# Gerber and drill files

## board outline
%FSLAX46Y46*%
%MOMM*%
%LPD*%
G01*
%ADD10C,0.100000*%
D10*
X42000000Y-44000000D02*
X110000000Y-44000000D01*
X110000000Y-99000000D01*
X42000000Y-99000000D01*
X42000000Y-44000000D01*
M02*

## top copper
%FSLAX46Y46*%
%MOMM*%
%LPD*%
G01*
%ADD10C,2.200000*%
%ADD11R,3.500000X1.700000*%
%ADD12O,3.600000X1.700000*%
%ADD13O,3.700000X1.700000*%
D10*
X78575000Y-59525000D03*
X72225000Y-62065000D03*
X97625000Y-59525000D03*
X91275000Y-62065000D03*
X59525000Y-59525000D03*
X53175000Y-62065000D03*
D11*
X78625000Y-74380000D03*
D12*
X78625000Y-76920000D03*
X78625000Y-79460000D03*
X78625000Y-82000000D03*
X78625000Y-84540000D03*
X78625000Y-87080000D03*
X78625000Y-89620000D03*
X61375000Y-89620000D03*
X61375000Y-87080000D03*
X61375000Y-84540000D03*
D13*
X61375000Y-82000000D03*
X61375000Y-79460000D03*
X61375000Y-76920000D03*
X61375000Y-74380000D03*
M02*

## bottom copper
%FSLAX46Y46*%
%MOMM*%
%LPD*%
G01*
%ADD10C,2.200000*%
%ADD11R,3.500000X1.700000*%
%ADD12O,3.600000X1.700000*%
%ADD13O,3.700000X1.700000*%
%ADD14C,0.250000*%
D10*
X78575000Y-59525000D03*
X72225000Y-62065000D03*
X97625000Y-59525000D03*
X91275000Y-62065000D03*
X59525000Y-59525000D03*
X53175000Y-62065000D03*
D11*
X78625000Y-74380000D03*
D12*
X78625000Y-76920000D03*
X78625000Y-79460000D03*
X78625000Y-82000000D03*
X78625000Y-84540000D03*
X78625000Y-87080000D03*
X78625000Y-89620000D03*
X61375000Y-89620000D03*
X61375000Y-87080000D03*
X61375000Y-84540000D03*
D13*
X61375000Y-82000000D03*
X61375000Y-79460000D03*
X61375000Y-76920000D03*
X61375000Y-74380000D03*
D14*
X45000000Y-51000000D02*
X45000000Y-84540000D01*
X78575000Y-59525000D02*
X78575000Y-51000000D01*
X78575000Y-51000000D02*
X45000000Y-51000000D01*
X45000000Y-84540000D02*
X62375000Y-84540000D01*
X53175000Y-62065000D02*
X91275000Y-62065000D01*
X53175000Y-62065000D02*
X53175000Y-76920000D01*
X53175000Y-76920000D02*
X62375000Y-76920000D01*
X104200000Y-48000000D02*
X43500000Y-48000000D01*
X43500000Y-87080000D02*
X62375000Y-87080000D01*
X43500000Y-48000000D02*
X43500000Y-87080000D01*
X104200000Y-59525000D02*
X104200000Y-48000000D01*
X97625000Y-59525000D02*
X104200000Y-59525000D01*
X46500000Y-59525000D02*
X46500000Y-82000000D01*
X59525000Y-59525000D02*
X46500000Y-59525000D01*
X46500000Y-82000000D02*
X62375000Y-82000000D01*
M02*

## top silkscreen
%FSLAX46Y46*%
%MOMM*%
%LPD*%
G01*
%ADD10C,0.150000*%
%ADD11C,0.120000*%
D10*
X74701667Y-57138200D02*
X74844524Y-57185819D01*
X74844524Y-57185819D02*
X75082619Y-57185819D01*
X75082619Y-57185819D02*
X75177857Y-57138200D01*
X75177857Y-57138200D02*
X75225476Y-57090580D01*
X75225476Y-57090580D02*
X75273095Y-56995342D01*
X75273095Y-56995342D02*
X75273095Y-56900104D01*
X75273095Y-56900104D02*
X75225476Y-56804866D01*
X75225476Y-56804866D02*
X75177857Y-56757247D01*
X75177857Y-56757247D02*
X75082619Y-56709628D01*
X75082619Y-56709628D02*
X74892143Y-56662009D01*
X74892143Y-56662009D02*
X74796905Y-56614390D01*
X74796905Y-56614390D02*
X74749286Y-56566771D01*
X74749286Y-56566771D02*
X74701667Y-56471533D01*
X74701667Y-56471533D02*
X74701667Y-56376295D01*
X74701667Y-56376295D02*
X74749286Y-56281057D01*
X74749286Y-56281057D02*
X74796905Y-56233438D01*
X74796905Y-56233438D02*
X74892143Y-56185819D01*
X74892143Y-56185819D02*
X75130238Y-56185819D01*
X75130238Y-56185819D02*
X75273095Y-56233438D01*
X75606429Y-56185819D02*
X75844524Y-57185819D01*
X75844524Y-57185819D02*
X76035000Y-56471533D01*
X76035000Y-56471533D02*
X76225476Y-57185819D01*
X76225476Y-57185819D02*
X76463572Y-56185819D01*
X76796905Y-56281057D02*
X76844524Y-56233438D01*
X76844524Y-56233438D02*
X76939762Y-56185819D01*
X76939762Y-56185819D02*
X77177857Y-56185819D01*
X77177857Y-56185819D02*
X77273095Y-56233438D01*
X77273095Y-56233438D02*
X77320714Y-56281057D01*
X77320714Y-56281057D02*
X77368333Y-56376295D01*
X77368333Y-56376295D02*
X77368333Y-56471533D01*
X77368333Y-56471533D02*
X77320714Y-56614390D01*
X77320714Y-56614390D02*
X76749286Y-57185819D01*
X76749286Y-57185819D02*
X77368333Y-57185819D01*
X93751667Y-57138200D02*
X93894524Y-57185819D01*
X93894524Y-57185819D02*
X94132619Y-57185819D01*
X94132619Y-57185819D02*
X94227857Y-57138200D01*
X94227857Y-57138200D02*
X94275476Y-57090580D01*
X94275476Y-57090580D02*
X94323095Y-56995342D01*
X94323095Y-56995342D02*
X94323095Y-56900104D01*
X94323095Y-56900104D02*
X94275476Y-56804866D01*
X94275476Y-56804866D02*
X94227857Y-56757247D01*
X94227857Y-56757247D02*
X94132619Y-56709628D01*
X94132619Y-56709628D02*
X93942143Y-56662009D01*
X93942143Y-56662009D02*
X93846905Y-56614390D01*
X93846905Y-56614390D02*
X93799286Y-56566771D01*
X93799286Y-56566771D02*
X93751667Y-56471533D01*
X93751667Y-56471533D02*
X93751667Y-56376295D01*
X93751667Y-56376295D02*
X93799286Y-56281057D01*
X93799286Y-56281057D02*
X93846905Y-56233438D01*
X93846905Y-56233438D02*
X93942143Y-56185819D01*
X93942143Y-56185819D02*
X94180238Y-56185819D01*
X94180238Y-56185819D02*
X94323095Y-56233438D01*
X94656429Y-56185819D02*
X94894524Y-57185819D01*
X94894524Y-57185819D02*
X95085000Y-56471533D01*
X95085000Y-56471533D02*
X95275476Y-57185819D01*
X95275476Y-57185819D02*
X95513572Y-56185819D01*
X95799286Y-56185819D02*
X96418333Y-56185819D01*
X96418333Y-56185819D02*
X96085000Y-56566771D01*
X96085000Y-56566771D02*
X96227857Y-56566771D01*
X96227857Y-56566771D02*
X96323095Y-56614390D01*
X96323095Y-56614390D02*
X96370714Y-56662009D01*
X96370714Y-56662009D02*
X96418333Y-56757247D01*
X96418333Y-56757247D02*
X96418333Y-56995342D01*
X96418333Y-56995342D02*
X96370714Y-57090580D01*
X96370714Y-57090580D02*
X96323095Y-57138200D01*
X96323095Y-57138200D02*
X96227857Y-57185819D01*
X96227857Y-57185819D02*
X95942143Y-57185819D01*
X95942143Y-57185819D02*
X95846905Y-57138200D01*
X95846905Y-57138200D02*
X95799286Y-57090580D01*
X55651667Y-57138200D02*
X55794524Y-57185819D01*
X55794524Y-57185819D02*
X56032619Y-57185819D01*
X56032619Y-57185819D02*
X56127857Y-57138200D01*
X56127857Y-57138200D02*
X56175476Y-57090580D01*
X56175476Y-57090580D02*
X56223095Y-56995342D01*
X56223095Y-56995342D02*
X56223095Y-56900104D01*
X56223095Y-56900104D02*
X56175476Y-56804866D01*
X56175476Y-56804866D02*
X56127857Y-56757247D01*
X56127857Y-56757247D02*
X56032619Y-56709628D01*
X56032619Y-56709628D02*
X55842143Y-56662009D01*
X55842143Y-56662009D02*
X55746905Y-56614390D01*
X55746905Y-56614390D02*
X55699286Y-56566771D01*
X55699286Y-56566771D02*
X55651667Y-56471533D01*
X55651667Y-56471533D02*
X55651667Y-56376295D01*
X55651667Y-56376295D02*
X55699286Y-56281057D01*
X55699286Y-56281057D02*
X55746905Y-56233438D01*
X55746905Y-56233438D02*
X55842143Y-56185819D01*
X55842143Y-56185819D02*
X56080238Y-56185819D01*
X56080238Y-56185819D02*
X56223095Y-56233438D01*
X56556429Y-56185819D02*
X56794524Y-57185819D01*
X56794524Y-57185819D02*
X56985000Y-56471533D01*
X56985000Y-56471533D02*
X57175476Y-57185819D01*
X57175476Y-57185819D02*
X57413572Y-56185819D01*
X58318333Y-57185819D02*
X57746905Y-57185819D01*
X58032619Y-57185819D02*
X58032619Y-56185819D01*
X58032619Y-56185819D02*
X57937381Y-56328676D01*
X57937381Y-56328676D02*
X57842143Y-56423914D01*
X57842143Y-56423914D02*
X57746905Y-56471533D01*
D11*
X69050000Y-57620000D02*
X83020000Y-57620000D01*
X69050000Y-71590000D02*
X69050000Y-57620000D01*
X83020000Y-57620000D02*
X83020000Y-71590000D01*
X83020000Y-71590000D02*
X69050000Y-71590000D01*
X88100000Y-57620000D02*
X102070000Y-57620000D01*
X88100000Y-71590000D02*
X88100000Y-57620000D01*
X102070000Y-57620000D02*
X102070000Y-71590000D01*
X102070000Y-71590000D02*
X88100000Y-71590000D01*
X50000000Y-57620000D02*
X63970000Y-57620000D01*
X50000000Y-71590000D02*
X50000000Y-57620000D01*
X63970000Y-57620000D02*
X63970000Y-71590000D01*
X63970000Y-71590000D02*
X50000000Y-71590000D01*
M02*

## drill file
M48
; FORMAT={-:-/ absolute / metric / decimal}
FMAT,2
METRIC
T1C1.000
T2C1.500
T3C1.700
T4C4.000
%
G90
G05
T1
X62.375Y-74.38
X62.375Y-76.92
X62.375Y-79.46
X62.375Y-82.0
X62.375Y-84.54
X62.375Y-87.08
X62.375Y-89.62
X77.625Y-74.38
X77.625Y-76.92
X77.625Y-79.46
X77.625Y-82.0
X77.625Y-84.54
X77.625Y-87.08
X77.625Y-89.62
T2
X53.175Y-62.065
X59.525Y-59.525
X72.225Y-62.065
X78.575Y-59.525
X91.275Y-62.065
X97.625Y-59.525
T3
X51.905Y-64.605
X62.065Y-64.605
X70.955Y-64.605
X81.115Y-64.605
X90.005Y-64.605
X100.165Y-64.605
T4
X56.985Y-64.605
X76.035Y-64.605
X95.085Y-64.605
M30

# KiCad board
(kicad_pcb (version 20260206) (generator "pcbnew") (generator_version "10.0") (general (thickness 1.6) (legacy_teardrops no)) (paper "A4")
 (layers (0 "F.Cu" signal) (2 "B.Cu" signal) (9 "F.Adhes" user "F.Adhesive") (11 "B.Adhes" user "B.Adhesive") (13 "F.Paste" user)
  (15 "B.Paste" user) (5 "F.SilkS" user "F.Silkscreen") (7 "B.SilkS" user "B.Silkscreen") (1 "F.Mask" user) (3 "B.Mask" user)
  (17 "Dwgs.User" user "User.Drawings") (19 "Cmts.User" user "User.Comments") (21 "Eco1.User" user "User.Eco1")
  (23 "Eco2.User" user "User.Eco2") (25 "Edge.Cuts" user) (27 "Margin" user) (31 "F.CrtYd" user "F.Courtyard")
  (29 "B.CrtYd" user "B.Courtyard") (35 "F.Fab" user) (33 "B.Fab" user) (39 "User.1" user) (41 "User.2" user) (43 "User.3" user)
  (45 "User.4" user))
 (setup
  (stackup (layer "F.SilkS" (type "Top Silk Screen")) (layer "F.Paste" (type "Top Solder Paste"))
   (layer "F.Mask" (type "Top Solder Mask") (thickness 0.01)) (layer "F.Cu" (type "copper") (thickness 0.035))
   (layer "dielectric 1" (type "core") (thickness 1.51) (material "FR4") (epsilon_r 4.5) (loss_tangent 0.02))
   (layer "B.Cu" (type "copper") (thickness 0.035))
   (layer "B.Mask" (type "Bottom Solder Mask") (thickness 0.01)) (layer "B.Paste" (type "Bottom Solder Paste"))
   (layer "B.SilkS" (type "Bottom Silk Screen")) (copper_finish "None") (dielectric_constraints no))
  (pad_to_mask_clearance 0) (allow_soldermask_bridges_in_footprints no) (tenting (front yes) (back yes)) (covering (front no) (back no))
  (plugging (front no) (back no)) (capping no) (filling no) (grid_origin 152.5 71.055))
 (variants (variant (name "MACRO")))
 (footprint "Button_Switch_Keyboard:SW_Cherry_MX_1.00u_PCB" (layer "F.Cu") (at 78.575 59.525)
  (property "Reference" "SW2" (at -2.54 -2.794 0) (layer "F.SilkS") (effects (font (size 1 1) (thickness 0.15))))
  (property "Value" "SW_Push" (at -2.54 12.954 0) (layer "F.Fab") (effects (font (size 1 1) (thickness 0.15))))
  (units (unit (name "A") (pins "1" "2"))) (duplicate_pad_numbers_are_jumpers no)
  (fp_line (start -9.525 -1.905) (end 4.445 -1.905) (stroke (width 0.12) (type solid)) (layer "F.SilkS"))
  (fp_line (start -9.525 12.065) (end -9.525 -1.905) (stroke (width 0.12) (type solid)) (layer "F.SilkS"))
  (fp_line (start 4.445 -1.905) (end 4.445 12.065) (stroke (width 0.12) (type solid)) (layer "F.SilkS"))
  (fp_line (start 4.445 12.065) (end -9.525 12.065) (stroke (width 0.12) (type solid)) (layer "F.SilkS"))
  (pad "" np_thru_hole circle (at -7.62 5.08) (size 1.7 1.7) (drill 1.7) (layers "*.Cu" "*.Mask"))
  (pad "" np_thru_hole circle (at -2.54 5.08) (size 4 4) (drill 4) (layers "*.Cu" "*.Mask"))
  (pad "" np_thru_hole circle (at 2.54 5.08) (size 1.7 1.7) (drill 1.7) (layers "*.Cu" "*.Mask"))
  (pad "1" thru_hole circle (at 0 0) (size 2.2 2.2) (drill 1.5) (layers "*.Cu" "*.Mask") (remove_unused_layers no)
   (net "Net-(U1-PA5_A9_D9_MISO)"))
  (pad "2" thru_hole circle (at -6.35 2.54) (size 2.2 2.2) (drill 1.5) (layers "*.Cu" "*.Mask") (remove_unused_layers no) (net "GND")))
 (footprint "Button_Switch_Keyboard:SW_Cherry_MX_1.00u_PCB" (layer "F.Cu") (at 97.625 59.525)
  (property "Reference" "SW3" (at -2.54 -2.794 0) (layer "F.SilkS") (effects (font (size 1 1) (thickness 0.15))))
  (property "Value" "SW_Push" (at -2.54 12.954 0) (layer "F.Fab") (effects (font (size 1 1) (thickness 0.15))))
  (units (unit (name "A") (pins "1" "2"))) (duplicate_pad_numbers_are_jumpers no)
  (fp_line (start -9.525 -1.905) (end 4.445 -1.905) (stroke (width 0.12) (type solid)) (layer "F.SilkS"))
  (fp_line (start -9.525 12.065) (end -9.525 -1.905) (stroke (width 0.12) (type solid)) (layer "F.SilkS"))
  (fp_line (start 4.445 -1.905) (end 4.445 12.065) (stroke (width 0.12) (type solid)) (layer "F.SilkS"))
  (fp_line (start 4.445 12.065) (end -9.525 12.065) (stroke (width 0.12) (type solid)) (layer "F.SilkS"))
  (pad "" np_thru_hole circle (at -7.62 5.08) (size 1.7 1.7) (drill 1.7) (layers "*.Cu" "*.Mask"))
  (pad "" np_thru_hole circle (at -2.54 5.08) (size 4 4) (drill 4) (layers "*.Cu" "*.Mask"))
  (pad "" np_thru_hole circle (at 2.54 5.08) (size 1.7 1.7) (drill 1.7) (layers "*.Cu" "*.Mask"))
  (pad "1" thru_hole circle (at 0 0) (size 2.2 2.2) (drill 1.5) (layers "*.Cu" "*.Mask") (remove_unused_layers no)
   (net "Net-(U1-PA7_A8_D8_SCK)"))
  (pad "2" thru_hole circle (at -6.35 2.54) (size 2.2 2.2) (drill 1.5) (layers "*.Cu" "*.Mask") (remove_unused_layers no) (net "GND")))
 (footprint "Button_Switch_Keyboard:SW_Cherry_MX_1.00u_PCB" (layer "F.Cu") (at 59.525 59.525)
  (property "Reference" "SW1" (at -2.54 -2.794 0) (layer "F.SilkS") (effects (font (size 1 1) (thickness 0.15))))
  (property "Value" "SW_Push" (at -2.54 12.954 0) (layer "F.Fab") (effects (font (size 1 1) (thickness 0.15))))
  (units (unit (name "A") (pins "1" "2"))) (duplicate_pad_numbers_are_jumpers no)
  (fp_line (start -9.525 -1.905) (end 4.445 -1.905) (stroke (width 0.12) (type solid)) (layer "F.SilkS"))
  (fp_line (start -9.525 12.065) (end -9.525 -1.905) (stroke (width 0.12) (type solid)) (layer "F.SilkS"))
  (fp_line (start 4.445 -1.905) (end 4.445 12.065) (stroke (width 0.12) (type solid)) (layer "F.SilkS"))
  (fp_line (start 4.445 12.065) (end -9.525 12.065) (stroke (width 0.12) (type solid)) (layer "F.SilkS"))
  (pad "" np_thru_hole circle (at -7.62 5.08) (size 1.7 1.7) (drill 1.7) (layers "*.Cu" "*.Mask"))
  (pad "" np_thru_hole circle (at -2.54 5.08) (size 4 4) (drill 4) (layers "*.Cu" "*.Mask"))
  (pad "" np_thru_hole circle (at 2.54 5.08) (size 1.7 1.7) (drill 1.7) (layers "*.Cu" "*.Mask"))
  (pad "1" thru_hole circle (at 0 0) (size 2.2 2.2) (drill 1.5) (layers "*.Cu" "*.Mask") (remove_unused_layers no)
   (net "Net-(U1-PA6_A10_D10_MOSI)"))
  (pad "2" thru_hole circle (at -6.35 2.54) (size 2.2 2.2) (drill 1.5) (layers "*.Cu" "*.Mask") (remove_unused_layers no) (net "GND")))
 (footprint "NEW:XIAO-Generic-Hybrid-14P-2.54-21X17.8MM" (layer "B.Cu") (at 70 82 180)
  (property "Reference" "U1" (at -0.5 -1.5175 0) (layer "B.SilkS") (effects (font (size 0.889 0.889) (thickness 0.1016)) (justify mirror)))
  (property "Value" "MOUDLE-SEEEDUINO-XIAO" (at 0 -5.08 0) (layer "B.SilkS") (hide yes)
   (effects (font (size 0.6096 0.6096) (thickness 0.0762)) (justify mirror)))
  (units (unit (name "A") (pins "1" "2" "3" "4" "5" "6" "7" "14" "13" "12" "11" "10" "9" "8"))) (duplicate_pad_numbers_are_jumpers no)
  (pad "1" thru_hole rect (at -7.625 7.62 180) (size 3.5 1.7) (drill 1 (offset -1 0)) (layers "*.Cu" "*.Mask") (remove_unused_layers no)
   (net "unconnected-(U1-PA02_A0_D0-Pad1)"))
  (pad "2" thru_hole oval (at -7.625 5.08 180) (size 3.6 1.7) (drill 1 (offset -1 0)) (layers "*.Cu" "*.Mask") (remove_unused_layers no)
   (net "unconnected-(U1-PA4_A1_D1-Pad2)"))
  (pad "3" thru_hole oval (at -7.625 2.54 180) (size 3.6 1.7) (drill 1 (offset -1 0)) (layers "*.Cu" "*.Mask") (remove_unused_layers no)
   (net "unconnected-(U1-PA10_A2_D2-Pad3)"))
  (pad "4" thru_hole oval (at -7.625 0 180) (size 3.6 1.7) (drill 1 (offset -1 0)) (layers "*.Cu" "*.Mask") (remove_unused_layers no)
   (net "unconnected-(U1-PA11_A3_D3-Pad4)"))
  (pad "5" thru_hole oval (at -7.625 -2.54 180) (size 3.6 1.7) (drill 1 (offset -1 0)) (layers "*.Cu" "*.Mask") (remove_unused_layers no)
   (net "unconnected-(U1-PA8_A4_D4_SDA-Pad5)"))
  (pad "6" thru_hole oval (at -7.625 -5.08) (size 3.6 1.7) (drill 1 (offset 1 0)) (layers "*.Cu" "*.Mask") (remove_unused_layers no)
   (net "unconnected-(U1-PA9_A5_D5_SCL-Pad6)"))
  (pad "7" thru_hole oval (at -7.625 -7.62 180) (size 3.6 1.7) (drill 1 (offset -1 0)) (layers "*.Cu" "*.Mask") (remove_unused_layers no)
   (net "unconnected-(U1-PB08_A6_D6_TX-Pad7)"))
  (pad "8" thru_hole oval (at 7.625 -7.62 180) (size 3.6 1.7) (drill 1 (offset 1 0)) (layers "*.Cu" "*.Mask") (remove_unused_layers no)
   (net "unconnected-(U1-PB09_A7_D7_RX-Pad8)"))
  (pad "9" thru_hole oval (at 7.625 -5.08 180) (size 3.6 1.7) (drill 1 (offset 1 0)) (layers "*.Cu" "*.Mask") (remove_unused_layers no)
   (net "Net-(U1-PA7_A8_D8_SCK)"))
  (pad "10" thru_hole oval (at 7.625 -2.54 180) (size 3.6 1.7) (drill 1 (offset 1 0)) (layers "*.Cu" "*.Mask") (remove_unused_layers no)
   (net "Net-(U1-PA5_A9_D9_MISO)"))
  (pad "11" thru_hole oval (at 7.625 0 180) (size 3.7 1.7) (drill 1 (offset 1 0)) (layers "*.Cu" "*.Mask") (remove_unused_layers no)
   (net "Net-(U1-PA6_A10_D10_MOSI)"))
  (pad "12" thru_hole oval (at 7.625 2.54 180) (size 3.7 1.7) (drill 1 (offset 1 0)) (layers "*.Cu" "*.Mask") (remove_unused_layers no)
   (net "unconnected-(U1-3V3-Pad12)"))
  (pad "13" thru_hole oval (at 7.625 5.08 180) (size 3.7 1.7) (drill 1 (offset 1 0)) (layers "*.Cu" "*.Mask") (remove_unused_layers no)
   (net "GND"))
  (pad "14" thru_hole oval (at 7.625 7.62 180) (size 3.7 1.7) (drill 1 (offset 1 0)) (layers "*.Cu" "*.Mask") (remove_unused_layers no)
   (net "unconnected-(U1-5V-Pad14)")))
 (gr_rect (start 42 44) (end 110 99) (stroke (width 0.1) (type default)) (fill no) (layer "Edge.Cuts"))
 (segment (start 45 51) (end 45 84.54) (width 0.25) (layer "B.Cu") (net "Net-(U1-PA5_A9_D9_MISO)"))
 (segment (start 78.575 59.525) (end 78.575 51) (width 0.25) (layer "B.Cu") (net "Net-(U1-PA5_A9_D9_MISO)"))
 (segment (start 78.575 51) (end 45 51) (width 0.25) (layer "B.Cu") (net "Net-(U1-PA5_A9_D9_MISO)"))
 (segment (start 45 84.54) (end 62.375 84.54) (width 0.25) (layer "B.Cu") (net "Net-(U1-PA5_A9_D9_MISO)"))
 (segment (start 53.175 62.065) (end 91.275 62.065) (width 0.25) (layer "B.Cu") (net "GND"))
 (segment (start 53.175 62.065) (end 53.175 76.92) (width 0.25) (layer "B.Cu") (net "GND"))
 (segment (start 53.175 76.92) (end 62.375 76.92) (width 0.25) (layer "B.Cu") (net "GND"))
 (segment (start 104.2 48) (end 43.5 48) (width 0.25) (layer "B.Cu") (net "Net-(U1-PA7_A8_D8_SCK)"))
 (segment (start 43.5 87.08) (end 62.375 87.08) (width 0.25) (layer "B.Cu") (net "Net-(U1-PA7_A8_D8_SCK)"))
 (segment (start 43.5 48) (end 43.5 87.08) (width 0.25) (layer "B.Cu") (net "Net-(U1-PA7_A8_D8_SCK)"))
 (segment (start 104.2 59.525) (end 104.2 48) (width 0.25) (layer "B.Cu") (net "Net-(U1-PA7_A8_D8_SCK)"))
 (segment (start 97.625 59.525) (end 104.2 59.525) (width 0.25) (layer "B.Cu") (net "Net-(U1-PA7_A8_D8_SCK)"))
 (segment (start 46.5 59.525) (end 46.5 82) (width 0.25) (layer "B.Cu") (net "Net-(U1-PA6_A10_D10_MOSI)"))
 (segment (start 59.525 59.525) (end 46.5 59.525) (width 0.25) (layer "B.Cu") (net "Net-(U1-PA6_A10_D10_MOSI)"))
 (segment (start 46.5 82) (end 62.375 82) (width 0.25) (layer "B.Cu") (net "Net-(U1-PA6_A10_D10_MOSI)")))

